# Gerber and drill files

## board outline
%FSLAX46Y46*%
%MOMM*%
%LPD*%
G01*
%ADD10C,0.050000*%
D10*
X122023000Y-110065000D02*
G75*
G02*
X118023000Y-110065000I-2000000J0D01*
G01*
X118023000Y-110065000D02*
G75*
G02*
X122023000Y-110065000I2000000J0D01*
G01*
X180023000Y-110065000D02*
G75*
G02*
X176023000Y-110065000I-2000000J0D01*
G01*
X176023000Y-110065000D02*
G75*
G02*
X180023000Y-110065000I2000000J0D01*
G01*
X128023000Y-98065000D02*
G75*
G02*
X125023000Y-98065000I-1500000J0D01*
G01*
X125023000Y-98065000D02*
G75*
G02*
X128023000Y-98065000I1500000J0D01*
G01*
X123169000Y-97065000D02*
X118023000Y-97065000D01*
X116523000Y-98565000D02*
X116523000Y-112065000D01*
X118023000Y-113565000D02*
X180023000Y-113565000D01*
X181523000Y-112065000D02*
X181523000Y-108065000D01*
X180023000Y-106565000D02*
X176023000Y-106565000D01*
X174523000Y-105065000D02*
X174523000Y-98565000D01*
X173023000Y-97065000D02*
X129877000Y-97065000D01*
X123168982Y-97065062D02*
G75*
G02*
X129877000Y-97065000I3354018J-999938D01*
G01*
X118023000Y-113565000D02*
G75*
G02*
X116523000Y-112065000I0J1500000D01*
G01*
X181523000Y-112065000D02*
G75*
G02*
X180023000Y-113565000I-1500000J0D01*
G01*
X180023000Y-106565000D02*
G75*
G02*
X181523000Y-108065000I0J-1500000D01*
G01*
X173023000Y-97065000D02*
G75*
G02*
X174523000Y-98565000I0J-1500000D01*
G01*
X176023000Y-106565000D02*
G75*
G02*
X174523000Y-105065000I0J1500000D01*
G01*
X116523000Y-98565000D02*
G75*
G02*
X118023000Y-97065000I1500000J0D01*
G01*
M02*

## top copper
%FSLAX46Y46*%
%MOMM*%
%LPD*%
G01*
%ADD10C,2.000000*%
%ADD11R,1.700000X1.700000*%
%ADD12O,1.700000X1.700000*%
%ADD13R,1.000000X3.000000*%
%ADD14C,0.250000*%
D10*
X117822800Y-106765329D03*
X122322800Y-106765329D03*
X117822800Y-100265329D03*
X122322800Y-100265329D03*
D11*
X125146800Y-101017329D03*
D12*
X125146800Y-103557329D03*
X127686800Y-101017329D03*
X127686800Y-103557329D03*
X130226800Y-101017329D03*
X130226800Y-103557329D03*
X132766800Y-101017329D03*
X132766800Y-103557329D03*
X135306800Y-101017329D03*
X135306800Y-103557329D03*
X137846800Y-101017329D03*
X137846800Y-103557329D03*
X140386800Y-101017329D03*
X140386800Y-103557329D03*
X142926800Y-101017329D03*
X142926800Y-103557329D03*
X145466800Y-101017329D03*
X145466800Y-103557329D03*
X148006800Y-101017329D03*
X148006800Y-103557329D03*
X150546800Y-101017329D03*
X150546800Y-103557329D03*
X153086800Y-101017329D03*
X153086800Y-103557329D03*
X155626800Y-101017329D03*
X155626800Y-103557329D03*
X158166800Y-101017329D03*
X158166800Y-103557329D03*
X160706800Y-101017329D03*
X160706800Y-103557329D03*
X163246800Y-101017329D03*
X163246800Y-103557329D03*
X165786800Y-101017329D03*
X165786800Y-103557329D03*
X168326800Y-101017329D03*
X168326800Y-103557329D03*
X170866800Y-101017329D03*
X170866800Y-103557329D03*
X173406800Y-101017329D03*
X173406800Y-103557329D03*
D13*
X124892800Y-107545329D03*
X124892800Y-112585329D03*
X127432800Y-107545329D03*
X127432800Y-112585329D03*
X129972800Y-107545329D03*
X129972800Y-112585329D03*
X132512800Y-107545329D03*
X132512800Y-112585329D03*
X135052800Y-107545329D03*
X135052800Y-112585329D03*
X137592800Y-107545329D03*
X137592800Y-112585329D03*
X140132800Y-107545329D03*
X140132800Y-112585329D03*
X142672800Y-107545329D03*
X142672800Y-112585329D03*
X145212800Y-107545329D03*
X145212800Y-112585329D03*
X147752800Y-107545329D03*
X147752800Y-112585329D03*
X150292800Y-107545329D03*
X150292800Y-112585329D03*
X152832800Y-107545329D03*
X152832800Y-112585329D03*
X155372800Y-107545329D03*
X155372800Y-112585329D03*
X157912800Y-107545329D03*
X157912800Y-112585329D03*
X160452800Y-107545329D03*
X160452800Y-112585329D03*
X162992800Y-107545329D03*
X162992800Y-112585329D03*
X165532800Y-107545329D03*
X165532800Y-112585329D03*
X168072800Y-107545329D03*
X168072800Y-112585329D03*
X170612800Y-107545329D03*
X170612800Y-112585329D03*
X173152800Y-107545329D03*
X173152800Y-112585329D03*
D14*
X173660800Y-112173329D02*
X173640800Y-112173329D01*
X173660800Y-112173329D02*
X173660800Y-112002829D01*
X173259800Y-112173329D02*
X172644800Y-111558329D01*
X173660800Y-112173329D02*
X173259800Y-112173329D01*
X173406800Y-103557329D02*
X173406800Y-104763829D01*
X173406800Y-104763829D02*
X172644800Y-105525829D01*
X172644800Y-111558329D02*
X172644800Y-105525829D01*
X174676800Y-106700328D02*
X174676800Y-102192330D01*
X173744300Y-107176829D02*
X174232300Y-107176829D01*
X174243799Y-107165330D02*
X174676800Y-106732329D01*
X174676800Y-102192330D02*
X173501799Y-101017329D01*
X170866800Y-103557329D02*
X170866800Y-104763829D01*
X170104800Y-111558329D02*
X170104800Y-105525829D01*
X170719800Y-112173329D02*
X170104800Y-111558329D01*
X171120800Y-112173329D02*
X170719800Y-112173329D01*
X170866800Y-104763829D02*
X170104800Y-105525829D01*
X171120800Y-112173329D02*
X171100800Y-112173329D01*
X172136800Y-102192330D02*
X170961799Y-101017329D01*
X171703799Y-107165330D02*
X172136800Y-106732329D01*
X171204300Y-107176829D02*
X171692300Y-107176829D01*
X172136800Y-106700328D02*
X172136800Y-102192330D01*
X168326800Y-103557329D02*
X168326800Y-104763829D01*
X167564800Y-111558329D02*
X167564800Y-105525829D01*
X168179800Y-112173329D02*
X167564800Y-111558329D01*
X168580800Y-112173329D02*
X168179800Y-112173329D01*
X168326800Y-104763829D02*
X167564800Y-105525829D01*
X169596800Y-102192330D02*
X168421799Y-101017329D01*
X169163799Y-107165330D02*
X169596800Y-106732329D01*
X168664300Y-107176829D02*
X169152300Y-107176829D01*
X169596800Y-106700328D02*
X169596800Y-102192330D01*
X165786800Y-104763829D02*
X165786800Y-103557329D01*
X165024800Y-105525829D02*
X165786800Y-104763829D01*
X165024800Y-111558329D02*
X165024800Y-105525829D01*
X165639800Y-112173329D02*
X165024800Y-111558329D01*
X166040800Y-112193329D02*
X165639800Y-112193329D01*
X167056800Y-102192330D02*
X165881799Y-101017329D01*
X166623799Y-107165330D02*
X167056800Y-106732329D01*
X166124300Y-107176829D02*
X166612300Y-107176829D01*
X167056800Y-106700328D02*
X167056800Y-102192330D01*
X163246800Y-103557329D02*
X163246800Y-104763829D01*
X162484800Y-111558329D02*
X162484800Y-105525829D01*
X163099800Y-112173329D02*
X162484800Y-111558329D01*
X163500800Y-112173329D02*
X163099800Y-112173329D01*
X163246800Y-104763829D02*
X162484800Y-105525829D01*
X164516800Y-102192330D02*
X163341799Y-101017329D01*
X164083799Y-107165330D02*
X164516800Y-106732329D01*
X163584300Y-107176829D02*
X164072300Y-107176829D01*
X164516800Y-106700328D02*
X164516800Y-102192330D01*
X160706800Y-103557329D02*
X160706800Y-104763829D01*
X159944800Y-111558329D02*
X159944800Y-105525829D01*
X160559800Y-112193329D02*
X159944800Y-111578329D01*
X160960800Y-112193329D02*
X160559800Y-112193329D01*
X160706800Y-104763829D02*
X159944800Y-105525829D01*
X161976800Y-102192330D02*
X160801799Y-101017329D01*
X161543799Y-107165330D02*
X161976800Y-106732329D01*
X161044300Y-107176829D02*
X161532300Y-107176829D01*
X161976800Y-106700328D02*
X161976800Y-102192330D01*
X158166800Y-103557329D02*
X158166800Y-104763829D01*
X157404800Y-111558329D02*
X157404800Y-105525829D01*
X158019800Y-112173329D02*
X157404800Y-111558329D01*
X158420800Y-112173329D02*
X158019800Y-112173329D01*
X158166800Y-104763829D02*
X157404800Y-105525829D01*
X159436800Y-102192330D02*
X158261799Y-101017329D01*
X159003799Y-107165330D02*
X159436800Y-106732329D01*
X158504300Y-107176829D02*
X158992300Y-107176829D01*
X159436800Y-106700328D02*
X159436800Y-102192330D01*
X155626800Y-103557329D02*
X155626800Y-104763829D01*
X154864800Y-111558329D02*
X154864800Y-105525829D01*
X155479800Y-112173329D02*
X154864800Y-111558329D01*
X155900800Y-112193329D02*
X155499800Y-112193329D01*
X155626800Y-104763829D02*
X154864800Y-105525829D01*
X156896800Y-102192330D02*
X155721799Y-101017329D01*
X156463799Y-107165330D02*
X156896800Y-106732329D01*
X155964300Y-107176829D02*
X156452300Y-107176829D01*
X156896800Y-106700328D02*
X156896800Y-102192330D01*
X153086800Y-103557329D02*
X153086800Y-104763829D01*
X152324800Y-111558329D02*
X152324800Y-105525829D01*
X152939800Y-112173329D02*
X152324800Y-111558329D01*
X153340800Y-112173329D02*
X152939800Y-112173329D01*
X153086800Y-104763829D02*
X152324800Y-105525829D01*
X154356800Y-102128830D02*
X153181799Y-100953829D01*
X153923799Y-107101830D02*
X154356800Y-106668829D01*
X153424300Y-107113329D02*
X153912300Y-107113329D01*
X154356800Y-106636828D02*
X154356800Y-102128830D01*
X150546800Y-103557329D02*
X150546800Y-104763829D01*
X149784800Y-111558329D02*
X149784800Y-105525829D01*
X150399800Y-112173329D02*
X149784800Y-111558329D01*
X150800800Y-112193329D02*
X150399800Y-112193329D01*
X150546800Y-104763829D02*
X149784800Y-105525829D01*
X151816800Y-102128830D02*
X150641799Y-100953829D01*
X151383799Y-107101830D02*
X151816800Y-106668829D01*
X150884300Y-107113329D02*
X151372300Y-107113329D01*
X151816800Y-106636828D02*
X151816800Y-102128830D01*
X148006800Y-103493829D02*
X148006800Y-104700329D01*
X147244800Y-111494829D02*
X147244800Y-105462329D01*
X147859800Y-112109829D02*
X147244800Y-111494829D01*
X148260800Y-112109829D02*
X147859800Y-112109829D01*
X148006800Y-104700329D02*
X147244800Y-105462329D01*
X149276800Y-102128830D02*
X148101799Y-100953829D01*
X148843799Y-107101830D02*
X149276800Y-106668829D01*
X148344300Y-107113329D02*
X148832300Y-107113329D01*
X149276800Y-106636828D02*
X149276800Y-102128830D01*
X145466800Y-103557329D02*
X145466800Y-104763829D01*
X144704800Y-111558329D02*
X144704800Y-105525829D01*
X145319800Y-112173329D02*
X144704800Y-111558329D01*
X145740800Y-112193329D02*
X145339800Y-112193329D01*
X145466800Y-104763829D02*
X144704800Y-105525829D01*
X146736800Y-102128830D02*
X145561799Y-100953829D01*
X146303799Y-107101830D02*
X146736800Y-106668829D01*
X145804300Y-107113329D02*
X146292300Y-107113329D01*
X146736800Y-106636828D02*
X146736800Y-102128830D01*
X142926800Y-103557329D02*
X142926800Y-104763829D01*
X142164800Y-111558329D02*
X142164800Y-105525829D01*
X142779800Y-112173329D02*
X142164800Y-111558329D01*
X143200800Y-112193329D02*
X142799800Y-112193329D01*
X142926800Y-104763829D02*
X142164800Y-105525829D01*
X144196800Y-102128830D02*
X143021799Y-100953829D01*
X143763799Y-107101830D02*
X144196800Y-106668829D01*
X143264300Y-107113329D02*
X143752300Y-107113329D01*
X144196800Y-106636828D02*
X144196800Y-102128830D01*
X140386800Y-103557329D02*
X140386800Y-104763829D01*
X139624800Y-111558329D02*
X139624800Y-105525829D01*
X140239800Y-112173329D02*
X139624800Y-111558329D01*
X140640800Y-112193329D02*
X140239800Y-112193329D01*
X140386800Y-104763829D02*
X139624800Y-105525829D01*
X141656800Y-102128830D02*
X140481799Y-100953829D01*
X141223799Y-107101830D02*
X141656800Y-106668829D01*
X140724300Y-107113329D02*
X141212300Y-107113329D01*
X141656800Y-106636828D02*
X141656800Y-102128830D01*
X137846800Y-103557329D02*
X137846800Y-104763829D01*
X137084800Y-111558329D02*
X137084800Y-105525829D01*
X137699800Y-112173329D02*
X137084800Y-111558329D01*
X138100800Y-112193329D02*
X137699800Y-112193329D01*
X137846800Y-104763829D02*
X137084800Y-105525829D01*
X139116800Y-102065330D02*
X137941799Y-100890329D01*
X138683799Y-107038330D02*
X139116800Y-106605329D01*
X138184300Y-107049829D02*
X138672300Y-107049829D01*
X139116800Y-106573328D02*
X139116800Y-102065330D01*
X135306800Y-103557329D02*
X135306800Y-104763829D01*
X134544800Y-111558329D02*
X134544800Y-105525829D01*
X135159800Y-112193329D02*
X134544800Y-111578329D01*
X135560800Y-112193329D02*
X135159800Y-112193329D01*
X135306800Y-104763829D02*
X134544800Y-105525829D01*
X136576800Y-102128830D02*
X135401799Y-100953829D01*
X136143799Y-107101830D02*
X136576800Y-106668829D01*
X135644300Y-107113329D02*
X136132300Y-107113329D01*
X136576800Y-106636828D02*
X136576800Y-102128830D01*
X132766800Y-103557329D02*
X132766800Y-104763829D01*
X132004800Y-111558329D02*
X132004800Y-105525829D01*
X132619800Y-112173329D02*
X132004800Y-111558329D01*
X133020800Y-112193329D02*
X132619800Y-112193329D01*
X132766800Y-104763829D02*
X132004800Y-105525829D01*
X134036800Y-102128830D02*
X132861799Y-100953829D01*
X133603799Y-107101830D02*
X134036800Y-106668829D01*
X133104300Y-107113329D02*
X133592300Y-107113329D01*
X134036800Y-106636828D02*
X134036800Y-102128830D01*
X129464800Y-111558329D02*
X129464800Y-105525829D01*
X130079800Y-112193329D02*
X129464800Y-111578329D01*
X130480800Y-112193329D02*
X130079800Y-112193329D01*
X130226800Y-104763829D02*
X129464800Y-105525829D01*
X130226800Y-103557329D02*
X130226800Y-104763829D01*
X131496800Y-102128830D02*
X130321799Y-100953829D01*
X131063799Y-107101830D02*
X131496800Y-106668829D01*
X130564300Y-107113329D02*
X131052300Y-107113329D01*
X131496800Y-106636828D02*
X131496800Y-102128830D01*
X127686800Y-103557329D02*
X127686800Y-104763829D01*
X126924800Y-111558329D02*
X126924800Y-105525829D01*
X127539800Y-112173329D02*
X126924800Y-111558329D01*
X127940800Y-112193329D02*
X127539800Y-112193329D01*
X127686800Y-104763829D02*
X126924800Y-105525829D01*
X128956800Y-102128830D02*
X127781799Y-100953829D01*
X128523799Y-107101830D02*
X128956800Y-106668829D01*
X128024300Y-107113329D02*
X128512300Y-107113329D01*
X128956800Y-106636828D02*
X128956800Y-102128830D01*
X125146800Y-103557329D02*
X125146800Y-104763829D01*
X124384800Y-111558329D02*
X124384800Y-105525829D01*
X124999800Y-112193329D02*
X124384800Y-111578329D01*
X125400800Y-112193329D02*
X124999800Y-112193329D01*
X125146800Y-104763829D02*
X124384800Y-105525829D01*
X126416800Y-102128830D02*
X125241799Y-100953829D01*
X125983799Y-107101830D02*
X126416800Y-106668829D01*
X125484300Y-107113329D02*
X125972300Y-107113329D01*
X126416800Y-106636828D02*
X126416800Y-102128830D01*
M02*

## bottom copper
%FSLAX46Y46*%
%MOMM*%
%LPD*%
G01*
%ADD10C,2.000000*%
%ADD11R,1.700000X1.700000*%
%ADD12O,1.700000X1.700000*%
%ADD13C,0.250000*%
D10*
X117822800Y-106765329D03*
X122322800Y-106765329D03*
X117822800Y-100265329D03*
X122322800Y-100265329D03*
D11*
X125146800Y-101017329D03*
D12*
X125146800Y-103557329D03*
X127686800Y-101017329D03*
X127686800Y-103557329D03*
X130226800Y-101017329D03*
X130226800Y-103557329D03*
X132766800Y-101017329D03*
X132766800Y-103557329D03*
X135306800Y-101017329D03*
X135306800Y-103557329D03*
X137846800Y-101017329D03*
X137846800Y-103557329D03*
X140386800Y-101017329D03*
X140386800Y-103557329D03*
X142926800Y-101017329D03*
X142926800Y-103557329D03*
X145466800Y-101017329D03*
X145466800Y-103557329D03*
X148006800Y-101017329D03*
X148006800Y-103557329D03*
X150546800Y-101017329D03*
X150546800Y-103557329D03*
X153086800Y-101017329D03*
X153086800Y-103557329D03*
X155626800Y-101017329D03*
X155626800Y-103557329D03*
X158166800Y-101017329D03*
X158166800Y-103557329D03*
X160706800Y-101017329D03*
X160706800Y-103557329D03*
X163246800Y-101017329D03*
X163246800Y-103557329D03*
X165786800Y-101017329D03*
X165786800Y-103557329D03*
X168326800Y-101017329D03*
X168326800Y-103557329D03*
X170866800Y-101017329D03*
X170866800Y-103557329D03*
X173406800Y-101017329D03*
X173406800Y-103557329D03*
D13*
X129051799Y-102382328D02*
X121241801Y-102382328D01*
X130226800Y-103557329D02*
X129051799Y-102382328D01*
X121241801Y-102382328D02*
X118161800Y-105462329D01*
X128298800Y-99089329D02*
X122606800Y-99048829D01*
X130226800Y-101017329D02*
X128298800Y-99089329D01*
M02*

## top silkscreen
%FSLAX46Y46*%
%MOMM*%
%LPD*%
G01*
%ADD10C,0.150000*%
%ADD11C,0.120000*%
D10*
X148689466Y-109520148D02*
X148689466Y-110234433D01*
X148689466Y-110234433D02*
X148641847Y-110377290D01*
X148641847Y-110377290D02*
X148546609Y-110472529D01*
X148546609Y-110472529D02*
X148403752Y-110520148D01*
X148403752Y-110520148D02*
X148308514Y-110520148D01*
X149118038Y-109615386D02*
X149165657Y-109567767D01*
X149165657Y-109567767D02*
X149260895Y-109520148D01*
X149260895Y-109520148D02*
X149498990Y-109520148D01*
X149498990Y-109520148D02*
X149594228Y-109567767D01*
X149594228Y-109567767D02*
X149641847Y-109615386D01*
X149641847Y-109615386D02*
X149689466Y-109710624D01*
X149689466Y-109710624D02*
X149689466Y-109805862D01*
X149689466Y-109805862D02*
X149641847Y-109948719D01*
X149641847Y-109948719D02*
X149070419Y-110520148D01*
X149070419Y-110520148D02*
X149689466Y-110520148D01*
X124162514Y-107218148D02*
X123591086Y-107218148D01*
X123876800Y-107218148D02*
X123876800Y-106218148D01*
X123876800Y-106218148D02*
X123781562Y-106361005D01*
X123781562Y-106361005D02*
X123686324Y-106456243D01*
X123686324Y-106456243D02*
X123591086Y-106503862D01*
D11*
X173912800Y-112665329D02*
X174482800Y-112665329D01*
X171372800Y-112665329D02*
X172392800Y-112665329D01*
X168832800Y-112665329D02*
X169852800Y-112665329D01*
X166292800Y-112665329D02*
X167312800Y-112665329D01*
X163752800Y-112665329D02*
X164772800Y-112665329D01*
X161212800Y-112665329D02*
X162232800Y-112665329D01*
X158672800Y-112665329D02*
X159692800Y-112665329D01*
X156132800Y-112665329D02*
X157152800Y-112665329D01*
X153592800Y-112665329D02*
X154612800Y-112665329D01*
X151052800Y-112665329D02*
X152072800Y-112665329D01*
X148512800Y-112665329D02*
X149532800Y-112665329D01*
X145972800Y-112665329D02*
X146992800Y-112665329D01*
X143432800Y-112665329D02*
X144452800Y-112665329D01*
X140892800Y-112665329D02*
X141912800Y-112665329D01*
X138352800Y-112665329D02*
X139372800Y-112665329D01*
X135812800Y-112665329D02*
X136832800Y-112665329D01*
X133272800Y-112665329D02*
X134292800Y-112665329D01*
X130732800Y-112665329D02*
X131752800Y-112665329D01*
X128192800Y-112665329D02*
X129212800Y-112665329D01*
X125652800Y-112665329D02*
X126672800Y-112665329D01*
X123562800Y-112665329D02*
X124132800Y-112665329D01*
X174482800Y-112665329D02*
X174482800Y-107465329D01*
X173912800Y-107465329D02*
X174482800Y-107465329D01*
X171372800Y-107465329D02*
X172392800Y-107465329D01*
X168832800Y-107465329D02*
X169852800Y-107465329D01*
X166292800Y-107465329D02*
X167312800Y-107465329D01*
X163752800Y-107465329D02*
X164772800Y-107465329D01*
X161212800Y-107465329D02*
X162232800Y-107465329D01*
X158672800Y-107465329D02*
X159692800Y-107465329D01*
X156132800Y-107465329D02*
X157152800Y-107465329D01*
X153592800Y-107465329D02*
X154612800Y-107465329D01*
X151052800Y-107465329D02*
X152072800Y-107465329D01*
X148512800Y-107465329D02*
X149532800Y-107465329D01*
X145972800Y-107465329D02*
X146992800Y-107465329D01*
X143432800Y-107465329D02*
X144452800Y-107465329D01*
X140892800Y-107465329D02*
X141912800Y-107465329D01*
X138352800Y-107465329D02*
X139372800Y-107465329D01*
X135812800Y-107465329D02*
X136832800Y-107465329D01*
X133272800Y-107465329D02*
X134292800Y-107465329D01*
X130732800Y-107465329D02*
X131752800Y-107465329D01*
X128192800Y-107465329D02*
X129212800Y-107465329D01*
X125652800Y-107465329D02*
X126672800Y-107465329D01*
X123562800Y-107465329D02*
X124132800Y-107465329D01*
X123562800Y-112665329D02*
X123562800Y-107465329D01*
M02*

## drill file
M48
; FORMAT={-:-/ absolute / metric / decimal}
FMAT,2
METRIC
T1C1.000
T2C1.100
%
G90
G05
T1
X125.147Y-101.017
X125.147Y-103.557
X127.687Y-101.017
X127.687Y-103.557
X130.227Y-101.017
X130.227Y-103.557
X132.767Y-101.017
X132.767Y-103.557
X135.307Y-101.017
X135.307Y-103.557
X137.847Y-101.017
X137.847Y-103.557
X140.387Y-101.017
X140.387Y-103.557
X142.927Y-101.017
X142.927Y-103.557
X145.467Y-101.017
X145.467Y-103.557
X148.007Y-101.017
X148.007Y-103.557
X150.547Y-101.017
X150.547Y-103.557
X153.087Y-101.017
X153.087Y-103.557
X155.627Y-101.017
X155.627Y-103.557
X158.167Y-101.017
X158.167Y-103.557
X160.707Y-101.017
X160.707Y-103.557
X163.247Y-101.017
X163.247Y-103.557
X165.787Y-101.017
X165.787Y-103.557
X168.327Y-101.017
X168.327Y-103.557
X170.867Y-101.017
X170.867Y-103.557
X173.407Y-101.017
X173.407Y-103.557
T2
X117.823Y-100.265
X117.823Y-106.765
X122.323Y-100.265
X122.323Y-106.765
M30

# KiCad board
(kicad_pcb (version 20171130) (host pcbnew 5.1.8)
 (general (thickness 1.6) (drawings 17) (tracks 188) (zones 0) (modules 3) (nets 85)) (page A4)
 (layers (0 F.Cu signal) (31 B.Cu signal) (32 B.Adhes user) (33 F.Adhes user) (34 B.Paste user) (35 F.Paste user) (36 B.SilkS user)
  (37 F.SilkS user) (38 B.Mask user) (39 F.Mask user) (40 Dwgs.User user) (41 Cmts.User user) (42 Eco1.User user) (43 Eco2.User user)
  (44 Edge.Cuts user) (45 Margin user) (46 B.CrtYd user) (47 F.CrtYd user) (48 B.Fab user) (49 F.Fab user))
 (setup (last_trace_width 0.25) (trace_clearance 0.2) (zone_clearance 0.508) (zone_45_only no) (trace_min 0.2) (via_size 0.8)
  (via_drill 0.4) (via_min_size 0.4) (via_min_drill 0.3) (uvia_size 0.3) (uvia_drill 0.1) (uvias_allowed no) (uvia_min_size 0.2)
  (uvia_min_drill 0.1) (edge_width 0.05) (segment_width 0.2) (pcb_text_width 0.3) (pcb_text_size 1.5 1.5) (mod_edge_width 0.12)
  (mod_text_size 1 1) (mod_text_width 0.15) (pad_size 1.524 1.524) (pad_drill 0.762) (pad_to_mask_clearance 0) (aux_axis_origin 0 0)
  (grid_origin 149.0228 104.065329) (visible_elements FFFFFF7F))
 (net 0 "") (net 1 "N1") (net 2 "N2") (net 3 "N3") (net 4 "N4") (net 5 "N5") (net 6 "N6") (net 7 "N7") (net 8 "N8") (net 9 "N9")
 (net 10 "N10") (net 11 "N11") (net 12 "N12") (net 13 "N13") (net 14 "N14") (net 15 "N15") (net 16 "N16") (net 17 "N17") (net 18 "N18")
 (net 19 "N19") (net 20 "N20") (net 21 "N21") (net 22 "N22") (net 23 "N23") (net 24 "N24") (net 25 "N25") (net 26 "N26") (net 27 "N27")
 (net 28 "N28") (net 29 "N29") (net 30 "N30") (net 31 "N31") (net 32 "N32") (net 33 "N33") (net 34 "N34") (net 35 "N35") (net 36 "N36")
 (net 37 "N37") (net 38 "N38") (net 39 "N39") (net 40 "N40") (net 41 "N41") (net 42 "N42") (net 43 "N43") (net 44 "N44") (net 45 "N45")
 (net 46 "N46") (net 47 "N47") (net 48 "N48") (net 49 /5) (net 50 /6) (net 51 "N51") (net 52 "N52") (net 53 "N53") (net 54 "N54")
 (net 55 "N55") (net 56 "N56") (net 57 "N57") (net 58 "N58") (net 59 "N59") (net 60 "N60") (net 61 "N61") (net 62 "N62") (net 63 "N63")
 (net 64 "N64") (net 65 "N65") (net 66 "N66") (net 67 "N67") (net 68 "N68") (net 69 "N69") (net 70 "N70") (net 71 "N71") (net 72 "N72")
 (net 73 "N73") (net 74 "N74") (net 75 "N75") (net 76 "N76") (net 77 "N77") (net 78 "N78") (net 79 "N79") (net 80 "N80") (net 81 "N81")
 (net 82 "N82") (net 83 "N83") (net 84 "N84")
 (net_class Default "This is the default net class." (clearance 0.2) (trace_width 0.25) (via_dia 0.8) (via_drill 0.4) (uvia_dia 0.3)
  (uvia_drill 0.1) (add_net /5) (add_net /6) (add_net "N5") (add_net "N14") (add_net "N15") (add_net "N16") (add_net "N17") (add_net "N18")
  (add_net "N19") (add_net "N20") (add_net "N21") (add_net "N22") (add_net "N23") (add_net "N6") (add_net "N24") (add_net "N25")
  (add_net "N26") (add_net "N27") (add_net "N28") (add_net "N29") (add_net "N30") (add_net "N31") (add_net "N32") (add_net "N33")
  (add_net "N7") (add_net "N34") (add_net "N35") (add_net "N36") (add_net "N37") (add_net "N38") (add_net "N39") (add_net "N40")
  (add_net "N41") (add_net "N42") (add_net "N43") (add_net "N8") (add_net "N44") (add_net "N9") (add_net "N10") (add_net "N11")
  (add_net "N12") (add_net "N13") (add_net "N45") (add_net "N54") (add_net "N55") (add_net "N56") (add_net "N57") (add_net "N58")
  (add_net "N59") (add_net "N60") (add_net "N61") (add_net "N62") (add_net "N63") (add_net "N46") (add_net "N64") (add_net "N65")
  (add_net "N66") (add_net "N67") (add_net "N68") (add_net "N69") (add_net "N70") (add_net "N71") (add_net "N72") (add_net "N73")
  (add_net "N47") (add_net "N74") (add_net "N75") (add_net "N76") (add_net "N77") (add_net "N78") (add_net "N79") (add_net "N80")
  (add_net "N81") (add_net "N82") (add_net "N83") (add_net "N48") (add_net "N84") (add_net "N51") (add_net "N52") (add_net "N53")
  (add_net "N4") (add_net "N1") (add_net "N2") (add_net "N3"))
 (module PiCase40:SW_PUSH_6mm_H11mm (layer B.Cu) (at 120.0228 103.565329 90)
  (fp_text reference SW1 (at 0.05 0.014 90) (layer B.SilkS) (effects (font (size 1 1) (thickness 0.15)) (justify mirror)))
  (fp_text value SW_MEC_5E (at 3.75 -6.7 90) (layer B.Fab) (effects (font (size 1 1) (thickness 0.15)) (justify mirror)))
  (pad 2 thru_hole circle (at -3.2 -2.2) (size 2 2) (drill 1.1) (layers *.Cu *.Mask) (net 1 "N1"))
  (pad 3 thru_hole circle (at -3.2 2.3) (size 2 2) (drill 1.1) (layers *.Cu *.Mask) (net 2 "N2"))
  (pad 4 thru_hole circle (at 3.3 -2.2) (size 2 2) (drill 1.1) (layers *.Cu *.Mask) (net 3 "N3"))
  (pad 1 thru_hole circle (at 3.3 2.3) (size 2 2) (drill 1.1) (layers *.Cu *.Mask) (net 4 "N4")))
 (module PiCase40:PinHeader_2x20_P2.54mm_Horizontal (layer B.Cu) (at 125.1468 101.017329 270)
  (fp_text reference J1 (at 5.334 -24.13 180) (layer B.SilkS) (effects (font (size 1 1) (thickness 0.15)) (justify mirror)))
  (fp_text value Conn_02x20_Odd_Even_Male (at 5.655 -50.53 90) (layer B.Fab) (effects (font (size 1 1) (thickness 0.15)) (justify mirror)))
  (pad 1 thru_hole rect (at 0 0 270) (size 1.7 1.7) (drill 1) (layers *.Cu *.Mask) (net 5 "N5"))
  (pad 2 thru_hole oval (at 2.54 0 270) (size 1.7 1.7) (drill 1) (layers *.Cu *.Mask) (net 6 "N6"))
  (pad 3 thru_hole oval (at 0 -2.54 270) (size 1.7 1.7) (drill 1) (layers *.Cu *.Mask) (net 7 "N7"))
  (pad 4 thru_hole oval (at 2.54 -2.54 270) (size 1.7 1.7) (drill 1) (layers *.Cu *.Mask) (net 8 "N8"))
  (pad 5 thru_hole oval (at 0 -5.08 270) (size 1.7 1.7) (drill 1) (layers *.Cu *.Mask) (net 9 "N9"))
  (pad 6 thru_hole oval (at 2.54 -5.08 270) (size 1.7 1.7) (drill 1) (layers *.Cu *.Mask) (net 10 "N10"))
  (pad 7 thru_hole oval (at 0 -7.62 270) (size 1.7 1.7) (drill 1) (layers *.Cu *.Mask) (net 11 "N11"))
  (pad 8 thru_hole oval (at 2.54 -7.62 270) (size 1.7 1.7) (drill 1) (layers *.Cu *.Mask) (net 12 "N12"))
  (pad 9 thru_hole oval (at 0 -10.16 270) (size 1.7 1.7) (drill 1) (layers *.Cu *.Mask) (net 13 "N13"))
  (pad 10 thru_hole oval (at 2.54 -10.16 270) (size 1.7 1.7) (drill 1) (layers *.Cu *.Mask) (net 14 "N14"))
  (pad 11 thru_hole oval (at 0 -12.7 270) (size 1.7 1.7) (drill 1) (layers *.Cu *.Mask) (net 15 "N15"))
  (pad 12 thru_hole oval (at 2.54 -12.7 270) (size 1.7 1.7) (drill 1) (layers *.Cu *.Mask) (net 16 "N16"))
  (pad 13 thru_hole oval (at 0 -15.24 270) (size 1.7 1.7) (drill 1) (layers *.Cu *.Mask) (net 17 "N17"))
  (pad 14 thru_hole oval (at 2.54 -15.24 270) (size 1.7 1.7) (drill 1) (layers *.Cu *.Mask) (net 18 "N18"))
  (pad 15 thru_hole oval (at 0 -17.78 270) (size 1.7 1.7) (drill 1) (layers *.Cu *.Mask) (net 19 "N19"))
  (pad 16 thru_hole oval (at 2.54 -17.78 270) (size 1.7 1.7) (drill 1) (layers *.Cu *.Mask) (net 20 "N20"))
  (pad 17 thru_hole oval (at 0 -20.32 270) (size 1.7 1.7) (drill 1) (layers *.Cu *.Mask) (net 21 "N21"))
  (pad 18 thru_hole oval (at 2.54 -20.32 270) (size 1.7 1.7) (drill 1) (layers *.Cu *.Mask) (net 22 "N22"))
  (pad 19 thru_hole oval (at 0 -22.86 270) (size 1.7 1.7) (drill 1) (layers *.Cu *.Mask) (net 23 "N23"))
  (pad 20 thru_hole oval (at 2.54 -22.86 270) (size 1.7 1.7) (drill 1) (layers *.Cu *.Mask) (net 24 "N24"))
  (pad 21 thru_hole oval (at 0 -25.4 270) (size 1.7 1.7) (drill 1) (layers *.Cu *.Mask) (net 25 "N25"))
  (pad 22 thru_hole oval (at 2.54 -25.4 270) (size 1.7 1.7) (drill 1) (layers *.Cu *.Mask) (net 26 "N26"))
  (pad 23 thru_hole oval (at 0 -27.94 270) (size 1.7 1.7) (drill 1) (layers *.Cu *.Mask) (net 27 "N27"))
  (pad 24 thru_hole oval (at 2.54 -27.94 270) (size 1.7 1.7) (drill 1) (layers *.Cu *.Mask) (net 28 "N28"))
  (pad 25 thru_hole oval (at 0 -30.48 270) (size 1.7 1.7) (drill 1) (layers *.Cu *.Mask) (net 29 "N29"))
  (pad 26 thru_hole oval (at 2.54 -30.48 270) (size 1.7 1.7) (drill 1) (layers *.Cu *.Mask) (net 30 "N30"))
  (pad 27 thru_hole oval (at 0 -33.02 270) (size 1.7 1.7) (drill 1) (layers *.Cu *.Mask) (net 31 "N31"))
  (pad 28 thru_hole oval (at 2.54 -33.02 270) (size 1.7 1.7) (drill 1) (layers *.Cu *.Mask) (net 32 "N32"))
  (pad 29 thru_hole oval (at 0 -35.56 270) (size 1.7 1.7) (drill 1) (layers *.Cu *.Mask) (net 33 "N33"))
  (pad 30 thru_hole oval (at 2.54 -35.56 270) (size 1.7 1.7) (drill 1) (layers *.Cu *.Mask) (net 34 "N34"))
  (pad 31 thru_hole oval (at 0 -38.1 270) (size 1.7 1.7) (drill 1) (layers *.Cu *.Mask) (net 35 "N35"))
  (pad 32 thru_hole oval (at 2.54 -38.1 270) (size 1.7 1.7) (drill 1) (layers *.Cu *.Mask) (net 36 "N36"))
  (pad 33 thru_hole oval (at 0 -40.64 270) (size 1.7 1.7) (drill 1) (layers *.Cu *.Mask) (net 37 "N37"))
  (pad 34 thru_hole oval (at 2.54 -40.64 270) (size 1.7 1.7) (drill 1) (layers *.Cu *.Mask) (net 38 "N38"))
  (pad 35 thru_hole oval (at 0 -43.18 270) (size 1.7 1.7) (drill 1) (layers *.Cu *.Mask) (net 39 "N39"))
  (pad 36 thru_hole oval (at 2.54 -43.18 270) (size 1.7 1.7) (drill 1) (layers *.Cu *.Mask) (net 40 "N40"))
  (pad 37 thru_hole oval (at 0 -45.72 270) (size 1.7 1.7) (drill 1) (layers *.Cu *.Mask) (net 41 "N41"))
  (pad 38 thru_hole oval (at 2.54 -45.72 270) (size 1.7 1.7) (drill 1) (layers *.Cu *.Mask) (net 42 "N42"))
  (pad 39 thru_hole oval (at 0 -48.26 270) (size 1.7 1.7) (drill 1) (layers *.Cu *.Mask) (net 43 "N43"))
  (pad 40 thru_hole oval (at 2.54 -48.26 270) (size 1.7 1.7) (drill 1) (layers *.Cu *.Mask) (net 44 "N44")))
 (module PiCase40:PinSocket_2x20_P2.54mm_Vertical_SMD (layer F.Cu) (at 149.0228 110.065329 90)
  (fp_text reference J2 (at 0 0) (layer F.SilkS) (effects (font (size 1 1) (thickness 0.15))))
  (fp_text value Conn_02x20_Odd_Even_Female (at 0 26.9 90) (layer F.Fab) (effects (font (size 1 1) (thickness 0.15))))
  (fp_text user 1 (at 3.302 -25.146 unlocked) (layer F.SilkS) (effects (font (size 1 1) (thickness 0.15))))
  (fp_line (start -2.6 24.89) (end -2.6 25.46) (layer F.SilkS) (width 0.12))
  (fp_line (start -2.6 22.35) (end -2.6 23.37) (layer F.SilkS) (width 0.12))
  (fp_line (start -2.6 19.81) (end -2.6 20.83) (layer F.SilkS) (width 0.12))
  (fp_line (start -2.6 17.27) (end -2.6 18.29) (layer F.SilkS) (width 0.12))
  (fp_line (start -2.6 14.73) (end -2.6 15.75) (layer F.SilkS) (width 0.12))
  (fp_line (start -2.6 12.19) (end -2.6 13.21) (layer F.SilkS) (width 0.12))
  (fp_line (start -2.6 9.65) (end -2.6 10.67) (layer F.SilkS) (width 0.12))
  (fp_line (start -2.6 7.11) (end -2.6 8.13) (layer F.SilkS) (width 0.12))
  (fp_line (start -2.6 4.57) (end -2.6 5.59) (layer F.SilkS) (width 0.12))
  (fp_line (start -2.6 2.03) (end -2.6 3.05) (layer F.SilkS) (width 0.12))
  (fp_line (start -2.6 -0.51) (end -2.6 0.51) (layer F.SilkS) (width 0.12))
  (fp_line (start -2.6 -3.05) (end -2.6 -2.03) (layer F.SilkS) (width 0.12))
  (fp_line (start -2.6 -5.59) (end -2.6 -4.57) (layer F.SilkS) (width 0.12))
  (fp_line (start -2.6 -8.13) (end -2.6 -7.11) (layer F.SilkS) (width 0.12))
  (fp_line (start -2.6 -10.67) (end -2.6 -9.65) (layer F.SilkS) (width 0.12))
  (fp_line (start -2.6 -13.21) (end -2.6 -12.19) (layer F.SilkS) (width 0.12))
  (fp_line (start -2.6 -15.75) (end -2.6 -14.73) (layer F.SilkS) (width 0.12))
  (fp_line (start -2.6 -18.29) (end -2.6 -17.27) (layer F.SilkS) (width 0.12))
  (fp_line (start -2.6 -20.83) (end -2.6 -19.81) (layer F.SilkS) (width 0.12))
  (fp_line (start -2.6 -23.37) (end -2.6 -22.35) (layer F.SilkS) (width 0.12))
  (fp_line (start -2.6 -25.46) (end -2.6 -24.89) (layer F.SilkS) (width 0.12))
  (fp_line (start -2.6 25.46) (end 2.6 25.46) (layer F.SilkS) (width 0.12))
  (fp_line (start 2.6 24.89) (end 2.6 25.46) (layer F.SilkS) (width 0.12))
  (fp_line (start 2.6 22.35) (end 2.6 23.37) (layer F.SilkS) (width 0.12))
  (fp_line (start 2.6 19.81) (end 2.6 20.83) (layer F.SilkS) (width 0.12))
  (fp_line (start 2.6 17.27) (end 2.6 18.29) (layer F.SilkS) (width 0.12))
  (fp_line (start 2.6 14.73) (end 2.6 15.75) (layer F.SilkS) (width 0.12))
  (fp_line (start 2.6 12.19) (end 2.6 13.21) (layer F.SilkS) (width 0.12))
  (fp_line (start 2.6 9.65) (end 2.6 10.67) (layer F.SilkS) (width 0.12))
  (fp_line (start 2.6 7.11) (end 2.6 8.13) (layer F.SilkS) (width 0.12))
  (fp_line (start 2.6 4.57) (end 2.6 5.59) (layer F.SilkS) (width 0.12))
  (fp_line (start 2.6 2.03) (end 2.6 3.05) (layer F.SilkS) (width 0.12))
  (fp_line (start 2.6 -0.51) (end 2.6 0.51) (layer F.SilkS) (width 0.12))
  (fp_line (start 2.6 -3.05) (end 2.6 -2.03) (layer F.SilkS) (width 0.12))
  (fp_line (start 2.6 -5.59) (end 2.6 -4.57) (layer F.SilkS) (width 0.12))
  (fp_line (start 2.6 -8.13) (end 2.6 -7.11) (layer F.SilkS) (width 0.12))
  (fp_line (start 2.6 -10.67) (end 2.6 -9.65) (layer F.SilkS) (width 0.12))
  (fp_line (start 2.6 -13.21) (end 2.6 -12.19) (layer F.SilkS) (width 0.12))
  (fp_line (start 2.6 -15.75) (end 2.6 -14.73) (layer F.SilkS) (width 0.12))
  (fp_line (start 2.6 -18.29) (end 2.6 -17.27) (layer F.SilkS) (width 0.12))
  (fp_line (start 2.6 -20.83) (end 2.6 -19.81) (layer F.SilkS) (width 0.12))
  (fp_line (start 2.6 -23.37) (end 2.6 -22.35) (layer F.SilkS) (width 0.12))
  (fp_line (start 2.6 -25.46) (end 2.6 -24.89) (layer F.SilkS) (width 0.12))
  (fp_line (start -2.6 -25.46) (end 2.6 -25.46) (layer F.SilkS) (width 0.12))
  (pad 1 smd rect (at 2.52 -24.13 90) (size 3 1) (layers F.Cu F.Paste F.Mask) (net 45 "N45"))
  (pad 2 smd rect (at -2.52 -24.13 90) (size 3 1) (layers F.Cu F.Paste F.Mask) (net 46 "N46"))
  (pad 3 smd rect (at 2.52 -21.59 90) (size 3 1) (layers F.Cu F.Paste F.Mask) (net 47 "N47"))
  (pad 4 smd rect (at -2.52 -21.59 90) (size 3 1) (layers F.Cu F.Paste F.Mask) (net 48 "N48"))
  (pad 5 smd rect (at 2.52 -19.05 90) (size 3 1) (layers F.Cu F.Paste F.Mask) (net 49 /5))
  (pad 6 smd rect (at -2.52 -19.05 90) (size 3 1) (layers F.Cu F.Paste F.Mask) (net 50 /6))
  (pad 7 smd rect (at 2.52 -16.51 90) (size 3 1) (layers F.Cu F.Paste F.Mask) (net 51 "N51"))
  (pad 8 smd rect (at -2.52 -16.51 90) (size 3 1) (layers F.Cu F.Paste F.Mask) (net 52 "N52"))
  (pad 9 smd rect (at 2.52 -13.97 90) (size 3 1) (layers F.Cu F.Paste F.Mask) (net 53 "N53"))
  (pad 10 smd rect (at -2.52 -13.97 90) (size 3 1) (layers F.Cu F.Paste F.Mask) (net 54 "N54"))
  (pad 11 smd rect (at 2.52 -11.43 90) (size 3 1) (layers F.Cu F.Paste F.Mask) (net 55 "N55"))
  (pad 12 smd rect (at -2.52 -11.43 90) (size 3 1) (layers F.Cu F.Paste F.Mask) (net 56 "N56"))
  (pad 13 smd rect (at 2.52 -8.89 90) (size 3 1) (layers F.Cu F.Paste F.Mask) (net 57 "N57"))
  (pad 14 smd rect (at -2.52 -8.89 90) (size 3 1) (layers F.Cu F.Paste F.Mask) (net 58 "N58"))
  (pad 15 smd rect (at 2.52 -6.35 90) (size 3 1) (layers F.Cu F.Paste F.Mask) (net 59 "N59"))
  (pad 16 smd rect (at -2.52 -6.35 90) (size 3 1) (layers F.Cu F.Paste F.Mask) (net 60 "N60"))
  (pad 17 smd rect (at 2.52 -3.81 90) (size 3 1) (layers F.Cu F.Paste F.Mask) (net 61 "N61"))
  (pad 18 smd rect (at -2.52 -3.81 90) (size 3 1) (layers F.Cu F.Paste F.Mask) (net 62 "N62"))
  (pad 19 smd rect (at 2.52 -1.27 90) (size 3 1) (layers F.Cu F.Paste F.Mask) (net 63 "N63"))
  (pad 20 smd rect (at -2.52 -1.27 90) (size 3 1) (layers F.Cu F.Paste F.Mask) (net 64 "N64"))
  (pad 21 smd rect (at 2.52 1.27 90) (size 3 1) (layers F.Cu F.Paste F.Mask) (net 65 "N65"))
  (pad 22 smd rect (at -2.52 1.27 90) (size 3 1) (layers F.Cu F.Paste F.Mask) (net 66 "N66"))
  (pad 23 smd rect (at 2.52 3.81 90) (size 3 1) (layers F.Cu F.Paste F.Mask) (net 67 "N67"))
  (pad 24 smd rect (at -2.52 3.81 90) (size 3 1) (layers F.Cu F.Paste F.Mask) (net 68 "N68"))
  (pad 25 smd rect (at 2.52 6.35 90) (size 3 1) (layers F.Cu F.Paste F.Mask) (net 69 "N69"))
  (pad 26 smd rect (at -2.52 6.35 90) (size 3 1) (layers F.Cu F.Paste F.Mask) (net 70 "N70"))
  (pad 27 smd rect (at 2.52 8.89 90) (size 3 1) (layers F.Cu F.Paste F.Mask) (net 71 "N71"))
  (pad 28 smd rect (at -2.52 8.89 90) (size 3 1) (layers F.Cu F.Paste F.Mask) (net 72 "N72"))
  (pad 29 smd rect (at 2.52 11.43 90) (size 3 1) (layers F.Cu F.Paste F.Mask) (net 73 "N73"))
  (pad 30 smd rect (at -2.52 11.43 90) (size 3 1) (layers F.Cu F.Paste F.Mask) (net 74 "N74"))
  (pad 31 smd rect (at 2.52 13.97 90) (size 3 1) (layers F.Cu F.Paste F.Mask) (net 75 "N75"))
  (pad 32 smd rect (at -2.52 13.97 90) (size 3 1) (layers F.Cu F.Paste F.Mask) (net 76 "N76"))
  (pad 33 smd rect (at 2.52 16.51 90) (size 3 1) (layers F.Cu F.Paste F.Mask) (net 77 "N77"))
  (pad 34 smd rect (at -2.52 16.51 90) (size 3 1) (layers F.Cu F.Paste F.Mask) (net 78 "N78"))
  (pad 35 smd rect (at 2.52 19.05 90) (size 3 1) (layers F.Cu F.Paste F.Mask) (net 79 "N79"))
  (pad 36 smd rect (at -2.52 19.05 90) (size 3 1) (layers F.Cu F.Paste F.Mask) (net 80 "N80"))
  (pad 37 smd rect (at 2.52 21.59 90) (size 3 1) (layers F.Cu F.Paste F.Mask) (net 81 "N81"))
  (pad 38 smd rect (at -2.52 21.59 90) (size 3 1) (layers F.Cu F.Paste F.Mask) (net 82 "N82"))
  (pad 39 smd rect (at 2.52 24.13 90) (size 3 1) (layers F.Cu F.Paste F.Mask) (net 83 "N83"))
  (pad 40 smd rect (at -2.52 24.13 90) (size 3 1) (layers F.Cu F.Paste F.Mask) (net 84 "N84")))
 (gr_circle (center 120.023 110.065) (end 118.023 110.065) (layer Edge.Cuts) (width 0.05))
 (gr_circle (center 178.023 110.065) (end 176.023 110.065) (layer Edge.Cuts) (width 0.05))
 (gr_circle (center 126.523 98.065) (end 125.023 98.065) (layer Edge.Cuts) (width 0.05))
 (gr_line (start 123.169 97.065) (end 118.023 97.065) (angle 90) (layer Edge.Cuts) (width 0.05))
 (gr_line (start 116.523 98.565) (end 116.523 112.065) (angle 90) (layer Edge.Cuts) (width 0.05))
 (gr_line (start 118.023 113.565) (end 180.023 113.565) (angle 90) (layer Edge.Cuts) (width 0.05))
 (gr_line (start 181.523 112.065) (end 181.523 108.065) (angle 90) (layer Edge.Cuts) (width 0.05))
 (gr_line (start 180.023 106.565) (end 176.023 106.565) (angle 90) (layer Edge.Cuts) (width 0.05))
 (gr_line (start 174.523 105.065) (end 174.523 98.565) (angle 90) (layer Edge.Cuts) (width 0.05))
 (gr_line (start 173.023 97.065) (end 129.877 97.065) (angle 90) (layer Edge.Cuts) (width 0.05))
 (gr_arc (start 126.523 98.065) (end 129.877 97.065) (angle -146.797) (layer Edge.Cuts) (width 0.05))
 (gr_arc (start 118.023 112.065) (end 116.523 112.065) (angle -90) (layer Edge.Cuts) (width 0.05))
 (gr_arc (start 180.023 112.065) (end 180.023 113.565) (angle -90) (layer Edge.Cuts) (width 0.05))
 (gr_arc (start 180.023 108.065) (end 181.523 108.065) (angle -90) (layer Edge.Cuts) (width 0.05))
 (gr_arc (start 173.023 98.565) (end 174.523 98.565) (angle -90) (layer Edge.Cuts) (width 0.05))
 (gr_arc (start 176.023 105.065) (end 174.523 105.065) (angle -90) (layer Edge.Cuts) (width 0.05))
 (gr_arc (start 118.023 98.565) (end 118.023 97.065) (angle -90) (layer Edge.Cuts) (width 0.05))
 (segment (start 173.6608 112.173329) (end 173.6408 112.173329) (width 0.25) (layer F.Cu) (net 44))
 (segment (start 173.6608 112.173329) (end 173.6608 112.002829) (width 0.25) (layer F.Cu) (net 44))
 (segment (start 173.2598 112.173329) (end 172.6448 111.558329) (width 0.25) (layer F.Cu) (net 44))
 (segment (start 173.6608 112.173329) (end 173.2598 112.173329) (width 0.25) (layer F.Cu) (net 44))
 (segment (start 173.4068 103.557329) (end 173.4068 104.763829) (width 0.25) (layer F.Cu) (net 44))
 (segment (start 173.4068 104.763829) (end 172.6448 105.525829) (width 0.25) (layer F.Cu) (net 44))
 (segment (start 172.6448 111.558329) (end 172.6448 105.525829) (width 0.25) (layer F.Cu) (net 44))
 (segment (start 174.6768 106.700328) (end 174.6768 102.19233) (width 0.25) (layer F.Cu) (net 43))
 (segment (start 173.7443 107.176829) (end 174.2323 107.176829) (width 0.25) (layer F.Cu) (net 43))
 (segment (start 174.243799 107.16533) (end 174.6768 106.732329) (width 0.25) (layer F.Cu) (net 43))
 (segment (start 174.6768 102.19233) (end 173.501799 101.017329) (width 0.25) (layer F.Cu) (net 43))
 (segment (start 170.8668 103.557329) (end 170.8668 104.763829) (width 0.25) (layer F.Cu) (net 42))
 (segment (start 170.1048 111.558329) (end 170.1048 105.525829) (width 0.25) (layer F.Cu) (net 42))
 (segment (start 170.7198 112.173329) (end 170.1048 111.558329) (width 0.25) (layer F.Cu) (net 42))
 (segment (start 171.1208 112.173329) (end 170.7198 112.173329) (width 0.25) (layer F.Cu) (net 42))
 (segment (start 170.8668 104.763829) (end 170.1048 105.525829) (width 0.25) (layer F.Cu) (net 42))
 (segment (start 171.1208 112.173329) (end 171.1008 112.173329) (width 0.25) (layer F.Cu) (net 42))
 (segment (start 172.1368 102.19233) (end 170.961799 101.017329) (width 0.25) (layer F.Cu) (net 41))
 (segment (start 171.703799 107.16533) (end 172.1368 106.732329) (width 0.25) (layer F.Cu) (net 41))
 (segment (start 171.2043 107.176829) (end 171.6923 107.176829) (width 0.25) (layer F.Cu) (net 41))
 (segment (start 172.1368 106.700328) (end 172.1368 102.19233) (width 0.25) (layer F.Cu) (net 41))
 (segment (start 168.3268 103.557329) (end 168.3268 104.763829) (width 0.25) (layer F.Cu) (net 40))
 (segment (start 167.5648 111.558329) (end 167.5648 105.525829) (width 0.25) (layer F.Cu) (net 40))
 (segment (start 168.1798 112.173329) (end 167.5648 111.558329) (width 0.25) (layer F.Cu) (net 40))
 (segment (start 168.5808 112.173329) (end 168.1798 112.173329) (width 0.25) (layer F.Cu) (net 40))
 (segment (start 168.3268 104.763829) (end 167.5648 105.525829) (width 0.25) (layer F.Cu) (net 40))
 (segment (start 169.5968 102.19233) (end 168.421799 101.017329) (width 0.25) (layer F.Cu) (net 39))
 (segment (start 169.163799 107.16533) (end 169.5968 106.732329) (width 0.25) (layer F.Cu) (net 39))
 (segment (start 168.6643 107.176829) (end 169.1523 107.176829) (width 0.25) (layer F.Cu) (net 39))
 (segment (start 169.5968 106.700328) (end 169.5968 102.19233) (width 0.25) (layer F.Cu) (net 39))
 (segment (start 165.7868 104.763829) (end 165.7868 103.557329) (width 0.25) (layer F.Cu) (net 38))
 (segment (start 165.0248 105.525829) (end 165.7868 104.763829) (width 0.25) (layer F.Cu) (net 38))
 (segment (start 165.0248 111.558329) (end 165.0248 105.525829) (width 0.25) (layer F.Cu) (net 38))
 (segment (start 165.6398 112.173329) (end 165.0248 111.558329) (width 0.25) (layer F.Cu) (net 38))
 (segment (start 166.0408 112.193329) (end 165.6398 112.193329) (width 0.25) (layer F.Cu) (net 38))
 (segment (start 167.0568 102.19233) (end 165.881799 101.017329) (width 0.25) (layer F.Cu) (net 37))
 (segment (start 166.623799 107.16533) (end 167.0568 106.732329) (width 0.25) (layer F.Cu) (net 37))
 (segment (start 166.1243 107.176829) (end 166.6123 107.176829) (width 0.25) (layer F.Cu) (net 37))
 (segment (start 167.0568 106.700328) (end 167.0568 102.19233) (width 0.25) (layer F.Cu) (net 37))
 (segment (start 163.2468 103.557329) (end 163.2468 104.763829) (width 0.25) (layer F.Cu) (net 36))
 (segment (start 162.4848 111.558329) (end 162.4848 105.525829) (width 0.25) (layer F.Cu) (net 36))
 (segment (start 163.0998 112.173329) (end 162.4848 111.558329) (width 0.25) (layer F.Cu) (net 36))
 (segment (start 163.5008 112.173329) (end 163.0998 112.173329) (width 0.25) (layer F.Cu) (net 36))
 (segment (start 163.2468 104.763829) (end 162.4848 105.525829) (width 0.25) (layer F.Cu) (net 36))
 (segment (start 164.5168 102.19233) (end 163.341799 101.017329) (width 0.25) (layer F.Cu) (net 35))
 (segment (start 164.083799 107.16533) (end 164.5168 106.732329) (width 0.25) (layer F.Cu) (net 35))
 (segment (start 163.5843 107.176829) (end 164.0723 107.176829) (width 0.25) (layer F.Cu) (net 35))
 (segment (start 164.5168 106.700328) (end 164.5168 102.19233) (width 0.25) (layer F.Cu) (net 35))
 (segment (start 160.7068 103.557329) (end 160.7068 104.763829) (width 0.25) (layer F.Cu) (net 34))
 (segment (start 159.9448 111.558329) (end 159.9448 105.525829) (width 0.25) (layer F.Cu) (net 34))
 (segment (start 160.5598 112.193329) (end 159.9448 111.578329) (width 0.25) (layer F.Cu) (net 34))
 (segment (start 160.9608 112.193329) (end 160.5598 112.193329) (width 0.25) (layer F.Cu) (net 34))
 (segment (start 160.7068 104.763829) (end 159.9448 105.525829) (width 0.25) (layer F.Cu) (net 34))
 (segment (start 161.9768 102.19233) (end 160.801799 101.017329) (width 0.25) (layer F.Cu) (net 33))
 (segment (start 161.543799 107.16533) (end 161.9768 106.732329) (width 0.25) (layer F.Cu) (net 33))
 (segment (start 161.0443 107.176829) (end 161.5323 107.176829) (width 0.25) (layer F.Cu) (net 33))
 (segment (start 161.9768 106.700328) (end 161.9768 102.19233) (width 0.25) (layer F.Cu) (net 33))
 (segment (start 158.1668 103.557329) (end 158.1668 104.763829) (width 0.25) (layer F.Cu) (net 32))
 (segment (start 157.4048 111.558329) (end 157.4048 105.525829) (width 0.25) (layer F.Cu) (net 32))
 (segment (start 158.0198 112.173329) (end 157.4048 111.558329) (width 0.25) (layer F.Cu) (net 32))
 (segment (start 158.4208 112.173329) (end 158.0198 112.173329) (width 0.25) (layer F.Cu) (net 32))
 (segment (start 158.1668 104.763829) (end 157.4048 105.525829) (width 0.25) (layer F.Cu) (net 32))
 (segment (start 159.4368 102.19233) (end 158.261799 101.017329) (width 0.25) (layer F.Cu) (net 31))
 (segment (start 159.003799 107.16533) (end 159.4368 106.732329) (width 0.25) (layer F.Cu) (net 31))
 (segment (start 158.5043 107.176829) (end 158.9923 107.176829) (width 0.25) (layer F.Cu) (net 31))
 (segment (start 159.4368 106.700328) (end 159.4368 102.19233) (width 0.25) (layer F.Cu) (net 31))
 (segment (start 155.6268 103.557329) (end 155.6268 104.763829) (width 0.25) (layer F.Cu) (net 30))
 (segment (start 154.8648 111.558329) (end 154.8648 105.525829) (width 0.25) (layer F.Cu) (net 30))
 (segment (start 155.4798 112.173329) (end 154.8648 111.558329) (width 0.25) (layer F.Cu) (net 30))
 (segment (start 155.9008 112.193329) (end 155.4998 112.193329) (width 0.25) (layer F.Cu) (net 30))
 (segment (start 155.6268 104.763829) (end 154.8648 105.525829) (width 0.25) (layer F.Cu) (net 30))
 (segment (start 156.8968 102.19233) (end 155.721799 101.017329) (width 0.25) (layer F.Cu) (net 29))
 (segment (start 156.463799 107.16533) (end 156.8968 106.732329) (width 0.25) (layer F.Cu) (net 29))
 (segment (start 155.9643 107.176829) (end 156.4523 107.176829) (width 0.25) (layer F.Cu) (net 29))
 (segment (start 156.8968 106.700328) (end 156.8968 102.19233) (width 0.25) (layer F.Cu) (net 29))
 (segment (start 153.0868 103.557329) (end 153.0868 104.763829) (width 0.25) (layer F.Cu) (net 28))
 (segment (start 152.3248 111.558329) (end 152.3248 105.525829) (width 0.25) (layer F.Cu) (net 28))
 (segment (start 152.9398 112.173329) (end 152.3248 111.558329) (width 0.25) (layer F.Cu) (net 28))
 (segment (start 153.3408 112.173329) (end 152.9398 112.173329) (width 0.25) (layer F.Cu) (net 28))
 (segment (start 153.0868 104.763829) (end 152.3248 105.525829) (width 0.25) (layer F.Cu) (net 28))
 (segment (start 154.3568 102.12883) (end 153.181799 100.953829) (width 0.25) (layer F.Cu) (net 27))
 (segment (start 153.923799 107.10183) (end 154.3568 106.668829) (width 0.25) (layer F.Cu) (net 27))
 (segment (start 153.4243 107.113329) (end 153.9123 107.113329) (width 0.25) (layer F.Cu) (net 27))
 (segment (start 154.3568 106.636828) (end 154.3568 102.12883) (width 0.25) (layer F.Cu) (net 27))
 (segment (start 150.5468 103.557329) (end 150.5468 104.763829) (width 0.25) (layer F.Cu) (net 26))
 (segment (start 149.7848 111.558329) (end 149.7848 105.525829) (width 0.25) (layer F.Cu) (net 26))
 (segment (start 150.3998 112.173329) (end 149.7848 111.558329) (width 0.25) (layer F.Cu) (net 26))
 (segment (start 150.8008 112.193329) (end 150.3998 112.193329) (width 0.25) (layer F.Cu) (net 26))
 (segment (start 150.5468 104.763829) (end 149.7848 105.525829) (width 0.25) (layer F.Cu) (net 26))
 (segment (start 151.8168 102.12883) (end 150.641799 100.953829) (width 0.25) (layer F.Cu) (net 25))
 (segment (start 151.383799 107.10183) (end 151.8168 106.668829) (width 0.25) (layer F.Cu) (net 25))
 (segment (start 150.8843 107.113329) (end 151.3723 107.113329) (width 0.25) (layer F.Cu) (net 25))
 (segment (start 151.8168 106.636828) (end 151.8168 102.12883) (width 0.25) (layer F.Cu) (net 25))
 (segment (start 148.0068 103.493829) (end 148.0068 104.700329) (width 0.25) (layer F.Cu) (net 24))
 (segment (start 147.2448 111.494829) (end 147.2448 105.462329) (width 0.25) (layer F.Cu) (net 24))
 (segment (start 147.8598 112.109829) (end 147.2448 111.494829) (width 0.25) (layer F.Cu) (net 24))
 (segment (start 148.2608 112.109829) (end 147.8598 112.109829) (width 0.25) (layer F.Cu) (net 24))
 (segment (start 148.0068 104.700329) (end 147.2448 105.462329) (width 0.25) (layer F.Cu) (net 24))
 (segment (start 149.2768 102.12883) (end 148.101799 100.953829) (width 0.25) (layer F.Cu) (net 23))
 (segment (start 148.843799 107.10183) (end 149.2768 106.668829) (width 0.25) (layer F.Cu) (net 23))
 (segment (start 148.3443 107.113329) (end 148.8323 107.113329) (width 0.25) (layer F.Cu) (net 23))
 (segment (start 149.2768 106.636828) (end 149.2768 102.12883) (width 0.25) (layer F.Cu) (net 23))
 (segment (start 145.4668 103.557329) (end 145.4668 104.763829) (width 0.25) (layer F.Cu) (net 22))
 (segment (start 144.7048 111.558329) (end 144.7048 105.525829) (width 0.25) (layer F.Cu) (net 22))
 (segment (start 145.3198 112.173329) (end 144.7048 111.558329) (width 0.25) (layer F.Cu) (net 22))
 (segment (start 145.7408 112.193329) (end 145.3398 112.193329) (width 0.25) (layer F.Cu) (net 22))
 (segment (start 145.4668 104.763829) (end 144.7048 105.525829) (width 0.25) (layer F.Cu) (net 22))
 (segment (start 146.7368 102.12883) (end 145.561799 100.953829) (width 0.25) (layer F.Cu) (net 21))
 (segment (start 146.303799 107.10183) (end 146.7368 106.668829) (width 0.25) (layer F.Cu) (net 21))
 (segment (start 145.8043 107.113329) (end 146.2923 107.113329) (width 0.25) (layer F.Cu) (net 21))
 (segment (start 146.7368 106.636828) (end 146.7368 102.12883) (width 0.25) (layer F.Cu) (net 21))
 (segment (start 142.9268 103.557329) (end 142.9268 104.763829) (width 0.25) (layer F.Cu) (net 20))
 (segment (start 142.1648 111.558329) (end 142.1648 105.525829) (width 0.25) (layer F.Cu) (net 20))
 (segment (start 142.7798 112.173329) (end 142.1648 111.558329) (width 0.25) (layer F.Cu) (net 20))
 (segment (start 143.2008 112.193329) (end 142.7998 112.193329) (width 0.25) (layer F.Cu) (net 20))
 (segment (start 142.9268 104.763829) (end 142.1648 105.525829) (width 0.25) (layer F.Cu) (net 20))
 (segment (start 144.1968 102.12883) (end 143.021799 100.953829) (width 0.25) (layer F.Cu) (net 19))
 (segment (start 143.763799 107.10183) (end 144.1968 106.668829) (width 0.25) (layer F.Cu) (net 19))
 (segment (start 143.2643 107.113329) (end 143.7523 107.113329) (width 0.25) (layer F.Cu) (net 19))
 (segment (start 144.1968 106.636828) (end 144.1968 102.12883) (width 0.25) (layer F.Cu) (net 19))
 (segment (start 140.3868 103.557329) (end 140.3868 104.763829) (width 0.25) (layer F.Cu) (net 18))
 (segment (start 139.6248 111.558329) (end 139.6248 105.525829) (width 0.25) (layer F.Cu) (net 18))
 (segment (start 140.2398 112.173329) (end 139.6248 111.558329) (width 0.25) (layer F.Cu) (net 18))
 (segment (start 140.6408 112.193329) (end 140.2398 112.193329) (width 0.25) (layer F.Cu) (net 18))
 (segment (start 140.3868 104.763829) (end 139.6248 105.525829) (width 0.25) (layer F.Cu) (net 18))
 (segment (start 141.6568 102.12883) (end 140.481799 100.953829) (width 0.25) (layer F.Cu) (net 17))
 (segment (start 141.223799 107.10183) (end 141.6568 106.668829) (width 0.25) (layer F.Cu) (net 17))
 (segment (start 140.7243 107.113329) (end 141.2123 107.113329) (width 0.25) (layer F.Cu) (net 17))
 (segment (start 141.6568 106.636828) (end 141.6568 102.12883) (width 0.25) (layer F.Cu) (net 17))
 (segment (start 137.8468 103.557329) (end 137.8468 104.763829) (width 0.25) (layer F.Cu) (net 16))
 (segment (start 137.0848 111.558329) (end 137.0848 105.525829) (width 0.25) (layer F.Cu) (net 16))
 (segment (start 137.6998 112.173329) (end 137.0848 111.558329) (width 0.25) (layer F.Cu) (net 16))
 (segment (start 138.1008 112.193329) (end 137.6998 112.193329) (width 0.25) (layer F.Cu) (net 16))
 (segment (start 137.8468 104.763829) (end 137.0848 105.525829) (width 0.25) (layer F.Cu) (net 16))
 (segment (start 139.1168 102.06533) (end 137.941799 100.890329) (width 0.25) (layer F.Cu) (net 15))
 (segment (start 138.683799 107.03833) (end 139.1168 106.605329) (width 0.25) (layer F.Cu) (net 15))
 (segment (start 138.1843 107.049829) (end 138.6723 107.049829) (width 0.25) (layer F.Cu) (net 15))
 (segment (start 139.1168 106.573328) (end 139.1168 102.06533) (width 0.25) (layer F.Cu) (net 15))
 (segment (start 135.3068 103.557329) (end 135.3068 104.763829) (width 0.25) (layer F.Cu) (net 14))
 (segment (start 134.5448 111.558329) (end 134.5448 105.525829) (width 0.25) (layer F.Cu) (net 14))
 (segment (start 135.1598 112.193329) (end 134.5448 111.578329) (width 0.25) (layer F.Cu) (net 14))
 (segment (start 135.5608 112.193329) (end 135.1598 112.193329) (width 0.25) (layer F.Cu) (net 14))
 (segment (start 135.3068 104.763829) (end 134.5448 105.525829) (width 0.25) (layer F.Cu) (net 14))
 (segment (start 136.5768 102.12883) (end 135.401799 100.953829) (width 0.25) (layer F.Cu) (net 13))
 (segment (start 136.143799 107.10183) (end 136.5768 106.668829) (width 0.25) (layer F.Cu) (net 13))
 (segment (start 135.6443 107.113329) (end 136.1323 107.113329) (width 0.25) (layer F.Cu) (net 13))
 (segment (start 136.5768 106.636828) (end 136.5768 102.12883) (width 0.25) (layer F.Cu) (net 13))
 (segment (start 132.7668 103.557329) (end 132.7668 104.763829) (width 0.25) (layer F.Cu) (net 12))
 (segment (start 132.0048 111.558329) (end 132.0048 105.525829) (width 0.25) (layer F.Cu) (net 12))
 (segment (start 132.6198 112.173329) (end 132.0048 111.558329) (width 0.25) (layer F.Cu) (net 12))
 (segment (start 133.0208 112.193329) (end 132.6198 112.193329) (width 0.25) (layer F.Cu) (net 12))
 (segment (start 132.7668 104.763829) (end 132.0048 105.525829) (width 0.25) (layer F.Cu) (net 12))
 (segment (start 134.0368 102.12883) (end 132.861799 100.953829) (width 0.25) (layer F.Cu) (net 11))
 (segment (start 133.603799 107.10183) (end 134.0368 106.668829) (width 0.25) (layer F.Cu) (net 11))
 (segment (start 133.1043 107.113329) (end 133.5923 107.113329) (width 0.25) (layer F.Cu) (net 11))
 (segment (start 134.0368 106.636828) (end 134.0368 102.12883) (width 0.25) (layer F.Cu) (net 11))
 (segment (start 129.4648 111.558329) (end 129.4648 105.525829) (width 0.25) (layer F.Cu) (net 50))
 (segment (start 130.0798 112.193329) (end 129.4648 111.578329) (width 0.25) (layer F.Cu) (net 50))
 (segment (start 130.4808 112.193329) (end 130.0798 112.193329) (width 0.25) (layer F.Cu) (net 50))
 (segment (start 130.2268 104.763829) (end 129.4648 105.525829) (width 0.25) (layer F.Cu) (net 50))
 (segment (start 130.2268 103.557329) (end 130.2268 104.763829) (width 0.25) (layer F.Cu) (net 50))
 (segment (start 129.051799 102.382328) (end 121.241801 102.382328) (width 0.25) (layer B.Cu) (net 50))
 (segment (start 130.2268 103.557329) (end 129.051799 102.382328) (width 0.25) (layer B.Cu) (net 50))
 (segment (start 121.241801 102.382328) (end 118.1618 105.462329) (width 0.25) (layer B.Cu) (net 50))
 (segment (start 131.4968 102.12883) (end 130.321799 100.953829) (width 0.25) (layer F.Cu) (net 9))
 (segment (start 131.063799 107.10183) (end 131.4968 106.668829) (width 0.25) (layer F.Cu) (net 9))
 (segment (start 130.5643 107.113329) (end 131.0523 107.113329) (width 0.25) (layer F.Cu) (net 9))
 (segment (start 131.4968 106.636828) (end 131.4968 102.12883) (width 0.25) (layer F.Cu) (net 9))
 (segment (start 128.2988 99.089329) (end 122.6068 99.048829) (width 0.25) (layer B.Cu) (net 9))
 (segment (start 130.2268 101.017329) (end 128.2988 99.089329) (width 0.25) (layer B.Cu) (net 9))
 (segment (start 127.6868 103.557329) (end 127.6868 104.763829) (width 0.25) (layer F.Cu) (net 8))
 (segment (start 126.9248 111.558329) (end 126.9248 105.525829) (width 0.25) (layer F.Cu) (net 8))
 (segment (start 127.5398 112.173329) (end 126.9248 111.558329) (width 0.25) (layer F.Cu) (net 8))
 (segment (start 127.9408 112.193329) (end 127.5398 112.193329) (width 0.25) (layer F.Cu) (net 8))
 (segment (start 127.6868 104.763829) (end 126.9248 105.525829) (width 0.25) (layer F.Cu) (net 8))
 (segment (start 128.9568 102.12883) (end 127.781799 100.953829) (width 0.25) (layer F.Cu) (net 7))
 (segment (start 128.523799 107.10183) (end 128.9568 106.668829) (width 0.25) (layer F.Cu) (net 7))
 (segment (start 128.0243 107.113329) (end 128.5123 107.113329) (width 0.25) (layer F.Cu) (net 7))
 (segment (start 128.9568 106.636828) (end 128.9568 102.12883) (width 0.25) (layer F.Cu) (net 7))
 (segment (start 125.1468 103.557329) (end 125.1468 104.763829) (width 0.25) (layer F.Cu) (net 6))
 (segment (start 124.3848 111.558329) (end 124.3848 105.525829) (width 0.25) (layer F.Cu) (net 6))
 (segment (start 124.9998 112.193329) (end 124.3848 111.578329) (width 0.25) (layer F.Cu) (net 6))
 (segment (start 125.4008 112.193329) (end 124.9998 112.193329) (width 0.25) (layer F.Cu) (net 6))
 (segment (start 125.1468 104.763829) (end 124.3848 105.525829) (width 0.25) (layer F.Cu) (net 6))
 (segment (start 126.4168 102.12883) (end 125.241799 100.953829) (width 0.25) (layer F.Cu) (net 5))
 (segment (start 125.983799 107.10183) (end 126.4168 106.668829) (width 0.25) (layer F.Cu) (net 5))
 (segment (start 125.4843 107.113329) (end 125.9723 107.113329) (width 0.25) (layer F.Cu) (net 5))
 (segment (start 126.4168 106.636828) (end 126.4168 102.12883) (width 0.25) (layer F.Cu) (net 5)))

